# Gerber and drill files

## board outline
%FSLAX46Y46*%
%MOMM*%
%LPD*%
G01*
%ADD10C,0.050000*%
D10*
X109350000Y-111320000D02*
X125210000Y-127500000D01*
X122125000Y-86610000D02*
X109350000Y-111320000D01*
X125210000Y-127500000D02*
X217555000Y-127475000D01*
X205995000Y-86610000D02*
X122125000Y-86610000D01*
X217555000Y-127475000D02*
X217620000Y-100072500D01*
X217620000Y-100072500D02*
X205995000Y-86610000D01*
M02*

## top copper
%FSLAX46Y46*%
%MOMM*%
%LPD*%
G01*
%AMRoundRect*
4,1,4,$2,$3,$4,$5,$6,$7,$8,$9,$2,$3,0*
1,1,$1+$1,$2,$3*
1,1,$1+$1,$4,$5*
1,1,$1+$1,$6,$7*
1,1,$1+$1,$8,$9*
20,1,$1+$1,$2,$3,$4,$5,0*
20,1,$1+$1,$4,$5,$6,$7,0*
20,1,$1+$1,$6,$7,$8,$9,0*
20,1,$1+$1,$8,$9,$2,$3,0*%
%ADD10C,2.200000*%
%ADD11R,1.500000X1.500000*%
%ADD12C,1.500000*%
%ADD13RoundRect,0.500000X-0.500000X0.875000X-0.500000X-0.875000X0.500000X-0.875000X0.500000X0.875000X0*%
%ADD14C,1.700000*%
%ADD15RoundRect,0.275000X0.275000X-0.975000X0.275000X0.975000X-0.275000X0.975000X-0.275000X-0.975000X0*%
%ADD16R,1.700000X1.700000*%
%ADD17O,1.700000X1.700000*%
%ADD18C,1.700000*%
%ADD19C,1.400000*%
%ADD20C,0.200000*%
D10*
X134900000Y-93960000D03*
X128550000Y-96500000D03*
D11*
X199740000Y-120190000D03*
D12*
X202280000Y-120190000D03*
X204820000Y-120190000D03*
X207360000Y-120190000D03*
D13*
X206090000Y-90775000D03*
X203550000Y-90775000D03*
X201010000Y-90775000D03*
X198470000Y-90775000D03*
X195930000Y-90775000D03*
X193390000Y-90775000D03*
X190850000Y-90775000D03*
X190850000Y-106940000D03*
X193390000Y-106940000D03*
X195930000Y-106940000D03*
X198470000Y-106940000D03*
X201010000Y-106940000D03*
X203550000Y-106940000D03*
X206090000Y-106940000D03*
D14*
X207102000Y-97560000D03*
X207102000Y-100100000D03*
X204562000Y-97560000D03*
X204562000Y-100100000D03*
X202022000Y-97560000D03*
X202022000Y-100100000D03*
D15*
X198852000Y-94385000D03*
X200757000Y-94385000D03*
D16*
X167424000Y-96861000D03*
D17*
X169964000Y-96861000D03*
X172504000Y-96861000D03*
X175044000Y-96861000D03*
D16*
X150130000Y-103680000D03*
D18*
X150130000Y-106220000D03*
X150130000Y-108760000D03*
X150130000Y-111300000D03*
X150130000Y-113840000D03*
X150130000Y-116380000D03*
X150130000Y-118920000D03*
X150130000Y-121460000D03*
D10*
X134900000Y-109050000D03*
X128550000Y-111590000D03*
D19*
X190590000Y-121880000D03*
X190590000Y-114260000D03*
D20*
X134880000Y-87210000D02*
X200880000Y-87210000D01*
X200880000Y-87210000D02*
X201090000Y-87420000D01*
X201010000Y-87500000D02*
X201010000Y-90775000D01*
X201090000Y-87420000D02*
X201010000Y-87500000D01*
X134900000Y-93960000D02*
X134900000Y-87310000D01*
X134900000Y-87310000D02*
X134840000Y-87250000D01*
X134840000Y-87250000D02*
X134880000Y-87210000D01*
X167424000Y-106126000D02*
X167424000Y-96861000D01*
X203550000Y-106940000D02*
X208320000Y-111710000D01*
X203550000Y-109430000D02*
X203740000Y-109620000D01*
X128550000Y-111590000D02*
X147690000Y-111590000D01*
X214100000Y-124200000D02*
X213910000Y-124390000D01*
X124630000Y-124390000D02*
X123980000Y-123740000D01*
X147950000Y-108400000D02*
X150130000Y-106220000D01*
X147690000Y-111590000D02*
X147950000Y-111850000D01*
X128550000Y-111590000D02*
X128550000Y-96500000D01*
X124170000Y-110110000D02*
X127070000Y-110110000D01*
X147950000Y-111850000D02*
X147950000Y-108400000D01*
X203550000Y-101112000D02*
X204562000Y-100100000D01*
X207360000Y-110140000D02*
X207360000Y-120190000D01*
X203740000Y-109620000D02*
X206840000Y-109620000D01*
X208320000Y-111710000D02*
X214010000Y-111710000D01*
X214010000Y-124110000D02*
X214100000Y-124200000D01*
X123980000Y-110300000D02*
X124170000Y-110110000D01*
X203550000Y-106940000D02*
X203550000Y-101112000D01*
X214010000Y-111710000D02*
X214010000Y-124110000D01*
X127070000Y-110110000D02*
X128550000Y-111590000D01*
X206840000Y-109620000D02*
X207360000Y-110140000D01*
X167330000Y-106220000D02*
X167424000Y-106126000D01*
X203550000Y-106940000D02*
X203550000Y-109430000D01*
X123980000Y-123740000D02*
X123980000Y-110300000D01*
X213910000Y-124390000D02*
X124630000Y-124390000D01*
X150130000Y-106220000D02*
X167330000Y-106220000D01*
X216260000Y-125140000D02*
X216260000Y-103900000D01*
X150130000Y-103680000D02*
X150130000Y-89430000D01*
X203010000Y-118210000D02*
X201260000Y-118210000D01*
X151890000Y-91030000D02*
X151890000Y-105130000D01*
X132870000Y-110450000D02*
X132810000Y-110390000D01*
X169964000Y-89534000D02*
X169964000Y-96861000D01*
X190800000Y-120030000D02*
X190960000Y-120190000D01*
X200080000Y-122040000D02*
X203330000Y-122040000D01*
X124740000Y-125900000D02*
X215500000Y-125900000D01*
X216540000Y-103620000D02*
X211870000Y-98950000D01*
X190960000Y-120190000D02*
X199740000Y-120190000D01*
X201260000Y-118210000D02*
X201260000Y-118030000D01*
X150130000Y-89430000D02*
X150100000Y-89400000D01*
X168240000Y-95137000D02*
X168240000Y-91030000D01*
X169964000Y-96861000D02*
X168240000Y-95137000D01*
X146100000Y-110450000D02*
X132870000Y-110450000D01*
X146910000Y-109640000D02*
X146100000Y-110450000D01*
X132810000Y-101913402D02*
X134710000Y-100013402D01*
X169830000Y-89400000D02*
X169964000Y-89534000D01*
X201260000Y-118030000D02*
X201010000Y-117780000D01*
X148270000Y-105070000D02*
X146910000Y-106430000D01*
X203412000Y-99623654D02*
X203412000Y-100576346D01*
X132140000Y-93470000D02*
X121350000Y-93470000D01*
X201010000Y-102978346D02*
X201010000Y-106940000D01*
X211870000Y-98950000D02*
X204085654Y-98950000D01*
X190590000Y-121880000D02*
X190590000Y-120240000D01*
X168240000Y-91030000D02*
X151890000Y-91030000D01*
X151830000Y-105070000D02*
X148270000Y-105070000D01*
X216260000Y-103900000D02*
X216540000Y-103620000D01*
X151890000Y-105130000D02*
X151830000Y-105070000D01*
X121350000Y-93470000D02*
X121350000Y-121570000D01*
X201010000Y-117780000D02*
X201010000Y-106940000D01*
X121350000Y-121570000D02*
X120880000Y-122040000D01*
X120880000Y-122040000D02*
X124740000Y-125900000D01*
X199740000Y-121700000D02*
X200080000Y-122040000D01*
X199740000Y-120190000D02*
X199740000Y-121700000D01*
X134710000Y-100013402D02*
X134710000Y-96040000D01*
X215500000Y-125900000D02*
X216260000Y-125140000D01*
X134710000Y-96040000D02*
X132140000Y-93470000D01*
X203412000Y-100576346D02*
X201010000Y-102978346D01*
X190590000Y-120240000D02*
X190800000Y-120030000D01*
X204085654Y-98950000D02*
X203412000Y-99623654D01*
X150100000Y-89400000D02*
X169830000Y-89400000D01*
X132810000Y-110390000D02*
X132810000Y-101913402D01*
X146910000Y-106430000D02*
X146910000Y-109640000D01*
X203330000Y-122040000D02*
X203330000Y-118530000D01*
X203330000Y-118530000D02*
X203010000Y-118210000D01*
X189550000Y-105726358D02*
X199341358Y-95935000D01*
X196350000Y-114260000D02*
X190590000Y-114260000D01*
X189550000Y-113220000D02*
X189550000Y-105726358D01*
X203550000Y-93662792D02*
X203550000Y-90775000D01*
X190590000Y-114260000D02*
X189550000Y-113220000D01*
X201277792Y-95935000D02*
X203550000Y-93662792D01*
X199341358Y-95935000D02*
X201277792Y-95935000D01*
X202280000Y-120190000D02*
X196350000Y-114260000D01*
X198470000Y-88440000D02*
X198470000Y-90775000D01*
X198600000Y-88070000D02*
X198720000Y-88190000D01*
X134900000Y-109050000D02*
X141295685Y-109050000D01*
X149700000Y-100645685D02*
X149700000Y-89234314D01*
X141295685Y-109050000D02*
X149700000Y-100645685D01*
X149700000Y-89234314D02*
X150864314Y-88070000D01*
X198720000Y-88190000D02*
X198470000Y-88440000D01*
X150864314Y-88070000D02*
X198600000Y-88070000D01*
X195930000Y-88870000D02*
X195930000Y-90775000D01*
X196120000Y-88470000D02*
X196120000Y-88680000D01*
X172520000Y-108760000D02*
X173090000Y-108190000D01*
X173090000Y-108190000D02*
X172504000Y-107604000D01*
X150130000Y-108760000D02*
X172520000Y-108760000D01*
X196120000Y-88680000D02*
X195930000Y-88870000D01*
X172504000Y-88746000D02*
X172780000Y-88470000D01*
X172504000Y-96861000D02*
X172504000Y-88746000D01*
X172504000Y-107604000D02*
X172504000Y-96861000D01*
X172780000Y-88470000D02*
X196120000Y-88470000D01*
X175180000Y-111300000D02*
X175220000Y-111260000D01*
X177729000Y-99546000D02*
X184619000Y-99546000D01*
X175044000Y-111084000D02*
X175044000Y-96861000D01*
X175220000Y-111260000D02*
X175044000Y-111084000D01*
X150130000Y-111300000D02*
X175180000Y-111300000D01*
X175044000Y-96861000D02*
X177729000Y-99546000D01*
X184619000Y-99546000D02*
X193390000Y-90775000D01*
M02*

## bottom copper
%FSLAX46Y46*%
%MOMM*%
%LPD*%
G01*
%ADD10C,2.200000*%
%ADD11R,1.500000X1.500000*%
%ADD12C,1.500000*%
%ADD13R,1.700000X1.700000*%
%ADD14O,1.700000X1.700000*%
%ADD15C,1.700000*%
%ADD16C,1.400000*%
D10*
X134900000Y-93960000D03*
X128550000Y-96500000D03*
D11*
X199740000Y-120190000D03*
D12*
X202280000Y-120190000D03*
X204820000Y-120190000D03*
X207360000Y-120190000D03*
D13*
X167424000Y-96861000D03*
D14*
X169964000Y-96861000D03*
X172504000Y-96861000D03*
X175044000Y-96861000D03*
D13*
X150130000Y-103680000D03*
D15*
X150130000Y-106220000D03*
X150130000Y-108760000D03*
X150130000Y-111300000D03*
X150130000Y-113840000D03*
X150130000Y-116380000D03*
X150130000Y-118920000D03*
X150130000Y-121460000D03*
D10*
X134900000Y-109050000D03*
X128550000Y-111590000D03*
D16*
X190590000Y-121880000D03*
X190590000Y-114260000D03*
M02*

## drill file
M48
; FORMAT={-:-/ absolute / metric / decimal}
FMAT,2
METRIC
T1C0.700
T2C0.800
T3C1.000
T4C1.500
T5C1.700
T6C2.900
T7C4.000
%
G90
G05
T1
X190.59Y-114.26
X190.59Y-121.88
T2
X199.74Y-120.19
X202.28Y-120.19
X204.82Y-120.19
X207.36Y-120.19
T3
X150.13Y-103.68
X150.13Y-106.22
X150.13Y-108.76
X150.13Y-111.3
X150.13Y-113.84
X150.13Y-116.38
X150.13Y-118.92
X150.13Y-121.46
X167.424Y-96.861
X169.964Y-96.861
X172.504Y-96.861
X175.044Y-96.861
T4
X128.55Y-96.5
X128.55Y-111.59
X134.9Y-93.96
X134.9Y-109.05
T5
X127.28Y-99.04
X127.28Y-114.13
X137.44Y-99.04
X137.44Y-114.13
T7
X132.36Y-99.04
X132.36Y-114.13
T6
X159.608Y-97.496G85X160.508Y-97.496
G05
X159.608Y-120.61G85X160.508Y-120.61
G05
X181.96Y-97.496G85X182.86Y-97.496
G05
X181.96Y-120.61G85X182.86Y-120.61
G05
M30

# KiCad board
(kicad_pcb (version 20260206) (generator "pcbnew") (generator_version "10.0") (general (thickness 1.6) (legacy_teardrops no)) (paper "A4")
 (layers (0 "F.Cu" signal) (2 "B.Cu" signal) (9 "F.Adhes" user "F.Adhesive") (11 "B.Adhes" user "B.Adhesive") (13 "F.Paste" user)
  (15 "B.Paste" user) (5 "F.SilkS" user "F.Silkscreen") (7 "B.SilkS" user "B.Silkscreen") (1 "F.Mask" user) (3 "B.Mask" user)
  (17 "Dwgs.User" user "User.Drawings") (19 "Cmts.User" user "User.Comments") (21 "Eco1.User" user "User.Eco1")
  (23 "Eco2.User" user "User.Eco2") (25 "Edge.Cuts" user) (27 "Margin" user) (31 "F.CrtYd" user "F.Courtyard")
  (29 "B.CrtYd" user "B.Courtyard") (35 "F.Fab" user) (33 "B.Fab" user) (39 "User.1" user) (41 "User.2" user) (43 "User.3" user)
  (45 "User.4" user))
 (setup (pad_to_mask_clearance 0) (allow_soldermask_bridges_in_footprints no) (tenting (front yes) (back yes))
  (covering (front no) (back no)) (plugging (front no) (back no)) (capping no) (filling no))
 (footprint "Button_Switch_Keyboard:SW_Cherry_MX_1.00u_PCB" (layer "F.Cu") (at 134.9 93.96)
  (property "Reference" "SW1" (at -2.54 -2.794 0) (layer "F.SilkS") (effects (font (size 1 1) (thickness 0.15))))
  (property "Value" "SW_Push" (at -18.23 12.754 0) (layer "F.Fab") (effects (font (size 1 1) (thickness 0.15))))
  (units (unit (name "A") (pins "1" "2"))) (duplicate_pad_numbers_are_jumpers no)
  (pad "" np_thru_hole circle (at -7.62 5.08) (size 1.7 1.7) (drill 1.7) (layers "*.Cu" "*.Mask"))
  (pad "" np_thru_hole circle (at -2.54 5.08) (size 4 4) (drill 4) (layers "*.Cu" "*.Mask"))
  (pad "" np_thru_hole circle (at 2.54 5.08) (size 1.7 1.7) (drill 1.7) (layers "*.Cu" "*.Mask"))
  (pad "1" thru_hole circle (at 0 0) (size 2.2 2.2) (drill 1.5) (layers "*.Cu" "*.Mask") (remove_unused_layers no) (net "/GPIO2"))
  (pad "2" thru_hole circle (at -6.35 2.54) (size 2.2 2.2) (drill 1.5) (layers "*.Cu" "*.Mask") (remove_unused_layers no) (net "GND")))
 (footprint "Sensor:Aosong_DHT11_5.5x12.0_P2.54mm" (layer "F.Cu") (at 199.74 120.19 90)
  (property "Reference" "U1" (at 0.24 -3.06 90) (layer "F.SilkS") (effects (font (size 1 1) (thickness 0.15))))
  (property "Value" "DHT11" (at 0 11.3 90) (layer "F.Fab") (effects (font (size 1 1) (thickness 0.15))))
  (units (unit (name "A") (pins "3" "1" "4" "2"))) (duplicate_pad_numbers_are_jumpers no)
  (pad "1" thru_hole rect (at 0 0 90) (size 1.5 1.5) (drill 0.8) (layers "*.Cu" "*.Mask") (remove_unused_layers no) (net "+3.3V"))
  (pad "2" thru_hole circle (at 0 2.54 90) (size 1.5 1.5) (drill 0.8) (layers "*.Cu" "*.Mask") (remove_unused_layers no) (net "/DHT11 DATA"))
  (pad "3" thru_hole circle (at 0 5.08 90) (size 1.5 1.5) (drill 0.8) (layers "*.Cu" "*.Mask") (remove_unused_layers no)
   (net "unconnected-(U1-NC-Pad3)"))
  (pad "4" thru_hole circle (at 0 7.62 90) (size 1.5 1.5) (drill 0.8) (layers "*.Cu" "*.Mask") (remove_unused_layers no) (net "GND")))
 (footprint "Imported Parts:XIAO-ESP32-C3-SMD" (layer "F.Cu") (at 187.97 89.94 -90)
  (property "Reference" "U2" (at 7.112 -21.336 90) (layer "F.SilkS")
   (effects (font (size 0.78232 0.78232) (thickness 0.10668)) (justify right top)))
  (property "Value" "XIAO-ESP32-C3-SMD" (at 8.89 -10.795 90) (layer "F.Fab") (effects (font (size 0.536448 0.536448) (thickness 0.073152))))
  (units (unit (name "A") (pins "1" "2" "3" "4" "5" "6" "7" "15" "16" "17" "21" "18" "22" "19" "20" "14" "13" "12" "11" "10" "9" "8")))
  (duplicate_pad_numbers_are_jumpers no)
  (pad "1" smd roundrect (at 0.835 -18.12 270) (size 2.75 2) (layers "F.Cu" "F.Mask" "F.Paste") (roundrect_rratio 0.25)
   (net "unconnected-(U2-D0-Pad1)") (solder_mask_margin 0.0508) (thermal_bridge_angle 45))
  (pad "2" smd roundrect (at 0.835 -15.58 270) (size 2.75 2) (layers "F.Cu" "F.Mask" "F.Paste") (roundrect_rratio 0.25) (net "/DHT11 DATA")
   (solder_mask_margin 0.0508) (thermal_bridge_angle 45))
  (pad "3" smd roundrect (at 0.835 -13.04 270) (size 2.75 2) (layers "F.Cu" "F.Mask" "F.Paste") (roundrect_rratio 0.25) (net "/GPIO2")
   (solder_mask_margin 0.0508) (thermal_bridge_angle 45))
  (pad "4" smd roundrect (at 0.835 -10.5 270) (size 2.75 2) (layers "F.Cu" "F.Mask" "F.Paste") (roundrect_rratio 0.25) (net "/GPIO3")
   (solder_mask_margin 0.0508) (thermal_bridge_angle 45))
  (pad "5" smd roundrect (at 0.835 -7.96 270) (size 2.75 2) (layers "F.Cu" "F.Mask" "F.Paste") (roundrect_rratio 0.25) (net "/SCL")
   (solder_mask_margin 0.0508) (thermal_bridge_angle 45))
  (pad "6" smd roundrect (at 0.835 -5.42 270) (size 2.75 2) (layers "F.Cu" "F.Mask" "F.Paste") (roundrect_rratio 0.25) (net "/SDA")
   (solder_mask_margin 0.0508) (thermal_bridge_angle 45))
  (pad "7" smd roundrect (at 0.835 -2.88 270) (size 2.75 2) (layers "F.Cu" "F.Mask" "F.Paste") (roundrect_rratio 0.25)
   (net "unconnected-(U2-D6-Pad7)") (solder_mask_margin 0.0508) (thermal_bridge_angle 45))
  (pad "8" smd roundrect (at 17 -2.88 270) (size 2.75 2) (layers "F.Cu" "F.Mask" "F.Paste") (roundrect_rratio 0.25)
   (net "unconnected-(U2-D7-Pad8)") (solder_mask_margin 0.0508) (thermal_bridge_angle 45))
  (pad "9" smd roundrect (at 17 -5.42 270) (size 2.75 2) (layers "F.Cu" "F.Mask" "F.Paste") (roundrect_rratio 0.25)
   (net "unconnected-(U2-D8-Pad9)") (solder_mask_margin 0.0508) (thermal_bridge_angle 45))
  (pad "10" smd roundrect (at 17 -7.96 270) (size 2.75 2) (layers "F.Cu" "F.Mask" "F.Paste") (roundrect_rratio 0.25)
   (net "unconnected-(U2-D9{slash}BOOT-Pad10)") (solder_mask_margin 0.0508) (thermal_bridge_angle 45))
  (pad "11" smd roundrect (at 17 -10.5 270) (size 2.75 2) (layers "F.Cu" "F.Mask" "F.Paste") (roundrect_rratio 0.25)
   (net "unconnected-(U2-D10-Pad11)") (solder_mask_margin 0.0508) (thermal_bridge_angle 45))
  (pad "12" smd roundrect (at 17 -13.04 270) (size 2.75 2) (layers "F.Cu" "F.Mask" "F.Paste") (roundrect_rratio 0.25) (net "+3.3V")
   (solder_mask_margin 0.0508) (thermal_bridge_angle 45))
  (pad "13" smd roundrect (at 17 -15.58 270) (size 2.75 2) (layers "F.Cu" "F.Mask" "F.Paste") (roundrect_rratio 0.25) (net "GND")
   (solder_mask_margin 0.0508) (thermal_bridge_angle 45))
  (pad "14" smd roundrect (at 17 -18.12 270) (size 2.75 2) (layers "F.Cu" "F.Mask" "F.Paste") (roundrect_rratio 0.25) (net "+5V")
   (solder_mask_margin 0.0508) (thermal_bridge_angle 45))
  (pad "15" smd circle (at 7.62 -19.132 270) (size 1.7 1.7) (layers "F.Cu" "F.Mask" "F.Paste") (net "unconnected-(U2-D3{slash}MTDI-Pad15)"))
  (pad "16" smd circle (at 10.16 -19.132 270) (size 1.7 1.7) (layers "F.Cu" "F.Mask" "F.Paste") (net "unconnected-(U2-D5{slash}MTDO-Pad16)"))
  (pad "17" smd circle (at 7.62 -16.592 270) (size 1.7 1.7) (layers "F.Cu" "F.Mask" "F.Paste") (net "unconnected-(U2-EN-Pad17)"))
  (pad "18" smd circle (at 10.16 -16.592 270) (size 1.7 1.7) (layers "F.Cu" "F.Mask" "F.Paste") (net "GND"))
  (pad "19" smd circle (at 7.62 -14.052 270) (size 1.7 1.7) (layers "F.Cu" "F.Mask" "F.Paste") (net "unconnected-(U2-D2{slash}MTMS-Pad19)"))
  (pad "20" smd circle (at 10.16 -14.052 270) (size 1.7 1.7) (layers "F.Cu" "F.Mask" "F.Paste") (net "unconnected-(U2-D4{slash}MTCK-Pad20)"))
  (pad "21" smd roundrect (at 4.445 -10.882 90) (size 2.5 1.1) (layers "F.Cu" "F.Mask" "F.Paste") (roundrect_rratio 0.25)
   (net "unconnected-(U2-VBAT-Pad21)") (thermal_bridge_angle 45))
  (pad "22" smd roundrect (at 4.445 -12.787 90) (size 2.5 1.1) (layers "F.Cu" "F.Mask" "F.Paste") (roundrect_rratio 0.25)
   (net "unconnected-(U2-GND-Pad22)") (thermal_bridge_angle 45)))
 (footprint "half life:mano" (layer "F.Cu") (at 180.8 111.37)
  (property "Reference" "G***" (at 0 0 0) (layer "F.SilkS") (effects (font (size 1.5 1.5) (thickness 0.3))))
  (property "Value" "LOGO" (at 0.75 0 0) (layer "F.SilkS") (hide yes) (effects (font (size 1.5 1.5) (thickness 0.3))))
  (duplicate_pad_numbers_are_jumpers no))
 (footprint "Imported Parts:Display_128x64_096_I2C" (layer "F.Cu") (at 171.234 96.861)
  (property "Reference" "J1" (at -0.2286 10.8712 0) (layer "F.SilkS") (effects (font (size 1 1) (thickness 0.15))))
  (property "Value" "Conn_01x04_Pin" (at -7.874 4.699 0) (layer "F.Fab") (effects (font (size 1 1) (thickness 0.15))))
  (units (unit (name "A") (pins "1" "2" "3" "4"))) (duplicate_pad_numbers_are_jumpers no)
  (pad "" np_thru_hole oval (at -11.176 0.635) (size 3.8 2.9) (drill oval 3.8 2.9) (layers "*.Cu" "*.Mask"))
  (pad "" np_thru_hole oval (at -11.176 23.749) (size 3.8 2.9) (drill oval 3.8 2.9) (layers "*.Cu" "*.Mask"))
  (pad "" np_thru_hole oval (at 11.176 0.635) (size 3.8 2.9) (drill oval 3.8 2.9) (layers "*.Cu" "*.Mask"))
  (pad "" np_thru_hole oval (at 11.176 23.749) (size 3.8 2.9) (drill oval 3.8 2.9) (layers "*.Cu" "*.Mask"))
  (pad "1" thru_hole rect (at -3.81 0 90) (size 1.7 1.7) (drill 1) (layers "*.Cu" "*.Mask") (remove_unused_layers no) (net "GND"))
  (pad "2" thru_hole oval (at -1.27 0 90) (size 1.7 1.7) (drill 1) (layers "*.Cu" "*.Mask") (remove_unused_layers no) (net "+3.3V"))
  (pad "3" thru_hole oval (at 1.27 0 90) (size 1.7 1.7) (drill 1) (layers "*.Cu" "*.Mask") (remove_unused_layers no) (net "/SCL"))
  (pad "4" thru_hole oval (at 3.81 0 90) (size 1.7 1.7) (drill 1) (layers "*.Cu" "*.Mask") (remove_unused_layers no) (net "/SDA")))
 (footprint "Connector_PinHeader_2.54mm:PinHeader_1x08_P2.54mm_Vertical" (layer "F.Cu") (at 150.13 103.68)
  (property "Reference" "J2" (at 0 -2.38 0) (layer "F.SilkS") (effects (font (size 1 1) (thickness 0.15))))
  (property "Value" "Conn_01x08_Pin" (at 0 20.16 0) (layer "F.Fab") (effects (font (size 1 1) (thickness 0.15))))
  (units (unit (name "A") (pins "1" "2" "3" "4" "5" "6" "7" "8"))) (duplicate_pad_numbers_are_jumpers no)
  (pad "1" thru_hole rect (at 0 0) (size 1.7 1.7) (drill 1) (layers "*.Cu" "*.Mask") (remove_unused_layers no) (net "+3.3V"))
  (pad "2" thru_hole circle (at 0 2.54) (size 1.7 1.7) (drill 1) (layers "*.Cu" "*.Mask") (remove_unused_layers no) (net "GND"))
  (pad "3" thru_hole circle (at 0 5.08) (size 1.7 1.7) (drill 1) (layers "*.Cu" "*.Mask") (remove_unused_layers no) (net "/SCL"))
  (pad "4" thru_hole circle (at 0 7.62) (size 1.7 1.7) (drill 1) (layers "*.Cu" "*.Mask") (remove_unused_layers no) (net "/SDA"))
  (pad "5" thru_hole circle (at 0 10.16) (size 1.7 1.7) (drill 1) (layers "*.Cu" "*.Mask") (remove_unused_layers no)
   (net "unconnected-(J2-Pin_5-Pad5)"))
  (pad "6" thru_hole circle (at 0 12.7) (size 1.7 1.7) (drill 1) (layers "*.Cu" "*.Mask") (remove_unused_layers no)
   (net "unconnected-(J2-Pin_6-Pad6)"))
  (pad "7" thru_hole circle (at 0 15.24) (size 1.7 1.7) (drill 1) (layers "*.Cu" "*.Mask") (remove_unused_layers no)
   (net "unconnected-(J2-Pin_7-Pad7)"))
  (pad "8" thru_hole circle (at 0 17.78) (size 1.7 1.7) (drill 1) (layers "*.Cu" "*.Mask") (remove_unused_layers no)
   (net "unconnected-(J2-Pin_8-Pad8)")))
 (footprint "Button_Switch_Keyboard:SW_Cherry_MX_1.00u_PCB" (layer "F.Cu") (at 134.9 109.05)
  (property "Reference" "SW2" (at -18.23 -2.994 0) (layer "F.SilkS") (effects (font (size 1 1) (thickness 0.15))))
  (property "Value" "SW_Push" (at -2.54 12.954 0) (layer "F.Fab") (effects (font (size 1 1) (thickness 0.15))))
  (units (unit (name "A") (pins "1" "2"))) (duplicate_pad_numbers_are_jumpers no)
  (pad "" np_thru_hole circle (at -7.62 5.08) (size 1.7 1.7) (drill 1.7) (layers "*.Cu" "*.Mask"))
  (pad "" np_thru_hole circle (at -2.54 5.08) (size 4 4) (drill 4) (layers "*.Cu" "*.Mask"))
  (pad "" np_thru_hole circle (at 2.54 5.08) (size 1.7 1.7) (drill 1.7) (layers "*.Cu" "*.Mask"))
  (pad "1" thru_hole circle (at 0 0) (size 2.2 2.2) (drill 1.5) (layers "*.Cu" "*.Mask") (remove_unused_layers no) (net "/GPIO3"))
  (pad "2" thru_hole circle (at -6.35 2.54) (size 2.2 2.2) (drill 1.5) (layers "*.Cu" "*.Mask") (remove_unused_layers no) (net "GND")))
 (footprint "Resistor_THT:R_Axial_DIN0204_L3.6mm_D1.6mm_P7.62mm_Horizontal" (layer "F.Cu") (at 190.59 121.88 90)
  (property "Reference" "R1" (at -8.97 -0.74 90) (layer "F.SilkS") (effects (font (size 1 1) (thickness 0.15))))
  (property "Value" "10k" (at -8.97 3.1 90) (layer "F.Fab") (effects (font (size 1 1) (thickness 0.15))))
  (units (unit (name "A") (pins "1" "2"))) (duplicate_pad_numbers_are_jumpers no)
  (pad "1" thru_hole circle (at 0 0 90) (size 1.4 1.4) (drill 0.7) (layers "*.Cu" "*.Mask") (remove_unused_layers no) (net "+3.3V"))
  (pad "2" thru_hole circle (at 7.62 0 90) (size 1.4 1.4) (drill 0.7) (layers "*.Cu" "*.Mask") (remove_unused_layers no) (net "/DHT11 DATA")))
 (gr_line (start 109.35 111.32) (end 125.21 127.5) (stroke (width 0.05) (type default)) (layer "Edge.Cuts"))
 (gr_line (start 122.125 86.61) (end 109.35 111.32) (stroke (width 0.05) (type default)) (layer "Edge.Cuts"))
 (gr_line (start 125.21 127.5) (end 217.555 127.475) (stroke (width 0.05) (type solid)) (layer "Edge.Cuts"))
 (gr_line (start 205.995 86.61) (end 122.125 86.61) (stroke (width 0.05) (type solid)) (layer "Edge.Cuts"))
 (gr_line (start 217.555 127.475) (end 217.62 100.0725) (stroke (width 0.05) (type solid)) (layer "Edge.Cuts"))
 (gr_line (start 217.62 100.0725) (end 205.995 86.61) (stroke (width 0.05) (type default)) (layer "Edge.Cuts"))
 (segment (start 134.88 87.21) (end 200.88 87.21) (width 0.2) (layer "F.Cu") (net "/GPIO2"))
 (segment (start 200.88 87.21) (end 201.09 87.42) (width 0.2) (layer "F.Cu") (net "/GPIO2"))
 (segment (start 201.01 87.5) (end 201.01 90.775) (width 0.2) (layer "F.Cu") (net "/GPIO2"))
 (segment (start 201.09 87.42) (end 201.01 87.5) (width 0.2) (layer "F.Cu") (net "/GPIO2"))
 (segment (start 134.9 93.96) (end 134.9 87.31) (width 0.2) (layer "F.Cu") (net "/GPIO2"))
 (segment (start 134.9 87.31) (end 134.84 87.25) (width 0.2) (layer "F.Cu") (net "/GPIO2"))
 (segment (start 134.84 87.25) (end 134.88 87.21) (width 0.2) (layer "F.Cu") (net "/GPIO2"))
 (segment (start 167.424 106.126) (end 167.424 96.861) (width 0.2) (layer "F.Cu") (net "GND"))
 (segment (start 203.55 106.94) (end 208.32 111.71) (width 0.2) (layer "F.Cu") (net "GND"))
 (segment (start 203.55 109.43) (end 203.74 109.62) (width 0.2) (layer "F.Cu") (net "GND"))
 (segment (start 128.55 111.59) (end 147.69 111.59) (width 0.2) (layer "F.Cu") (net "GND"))
 (segment (start 214.1 124.2) (end 213.91 124.39) (width 0.2) (layer "F.Cu") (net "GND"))
 (segment (start 124.63 124.39) (end 123.98 123.74) (width 0.2) (layer "F.Cu") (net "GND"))
 (segment (start 147.95 108.4) (end 150.13 106.22) (width 0.2) (layer "F.Cu") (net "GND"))
 (segment (start 147.69 111.59) (end 147.95 111.85) (width 0.2) (layer "F.Cu") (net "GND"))
 (segment (start 128.55 111.59) (end 128.55 96.5) (width 0.2) (layer "F.Cu") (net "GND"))
 (segment (start 124.17 110.11) (end 127.07 110.11) (width 0.2) (layer "F.Cu") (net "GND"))
 (segment (start 147.95 111.85) (end 147.95 108.4) (width 0.2) (layer "F.Cu") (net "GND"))
 (segment (start 203.55 101.112) (end 204.562 100.1) (width 0.2) (layer "F.Cu") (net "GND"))
 (segment (start 207.36 110.14) (end 207.36 120.19) (width 0.2) (layer "F.Cu") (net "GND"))
 (segment (start 203.74 109.62) (end 206.84 109.62) (width 0.2) (layer "F.Cu") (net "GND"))
 (segment (start 208.32 111.71) (end 214.01 111.71) (width 0.2) (layer "F.Cu") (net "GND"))
 (segment (start 214.01 124.11) (end 214.1 124.2) (width 0.2) (layer "F.Cu") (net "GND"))
 (segment (start 123.98 110.3) (end 124.17 110.11) (width 0.2) (layer "F.Cu") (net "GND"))
 (segment (start 203.55 106.94) (end 203.55 101.112) (width 0.2) (layer "F.Cu") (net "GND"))
 (segment (start 214.01 111.71) (end 214.01 124.11) (width 0.2) (layer "F.Cu") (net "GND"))
 (segment (start 127.07 110.11) (end 128.55 111.59) (width 0.2) (layer "F.Cu") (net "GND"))
 (segment (start 206.84 109.62) (end 207.36 110.14) (width 0.2) (layer "F.Cu") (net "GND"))
 (segment (start 167.33 106.22) (end 167.424 106.126) (width 0.2) (layer "F.Cu") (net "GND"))
 (segment (start 203.55 106.94) (end 203.55 109.43) (width 0.2) (layer "F.Cu") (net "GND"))
 (segment (start 123.98 123.74) (end 123.98 110.3) (width 0.2) (layer "F.Cu") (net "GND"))
 (segment (start 213.91 124.39) (end 124.63 124.39) (width 0.2) (layer "F.Cu") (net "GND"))
 (segment (start 150.13 106.22) (end 167.33 106.22) (width 0.2) (layer "F.Cu") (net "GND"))
 (segment (start 216.26 125.14) (end 216.26 103.9) (width 0.2) (layer "F.Cu") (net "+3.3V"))
 (segment (start 150.13 103.68) (end 150.13 89.43) (width 0.2) (layer "F.Cu") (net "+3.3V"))
 (segment (start 203.01 118.21) (end 201.26 118.21) (width 0.2) (layer "F.Cu") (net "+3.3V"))
 (segment (start 151.89 91.03) (end 151.89 105.13) (width 0.2) (layer "F.Cu") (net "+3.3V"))
 (segment (start 132.87 110.45) (end 132.81 110.39) (width 0.2) (layer "F.Cu") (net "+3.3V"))
 (segment (start 169.964 89.534) (end 169.964 96.861) (width 0.2) (layer "F.Cu") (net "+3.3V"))
 (segment (start 190.8 120.03) (end 190.96 120.19) (width 0.2) (layer "F.Cu") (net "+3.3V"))
 (segment (start 200.08 122.04) (end 203.33 122.04) (width 0.2) (layer "F.Cu") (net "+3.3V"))
 (segment (start 124.74 125.9) (end 215.5 125.9) (width 0.2) (layer "F.Cu") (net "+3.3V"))
 (segment (start 216.54 103.62) (end 211.87 98.95) (width 0.2) (layer "F.Cu") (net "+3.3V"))
 (segment (start 190.96 120.19) (end 199.74 120.19) (width 0.2) (layer "F.Cu") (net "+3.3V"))
 (segment (start 201.26 118.21) (end 201.26 118.03) (width 0.2) (layer "F.Cu") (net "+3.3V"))
 (segment (start 150.13 89.43) (end 150.1 89.4) (width 0.2) (layer "F.Cu") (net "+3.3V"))
 (segment (start 168.24 95.137) (end 168.24 91.03) (width 0.2) (layer "F.Cu") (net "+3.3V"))
 (segment (start 169.964 96.861) (end 168.24 95.137) (width 0.2) (layer "F.Cu") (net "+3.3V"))
 (segment (start 146.1 110.45) (end 132.87 110.45) (width 0.2) (layer "F.Cu") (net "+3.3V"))
 (segment (start 146.91 109.64) (end 146.1 110.45) (width 0.2) (layer "F.Cu") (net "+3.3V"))
 (segment (start 132.81 101.913402) (end 134.71 100.013402) (width 0.2) (layer "F.Cu") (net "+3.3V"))
 (segment (start 169.83 89.4) (end 169.964 89.534) (width 0.2) (layer "F.Cu") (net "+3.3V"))
 (segment (start 201.26 118.03) (end 201.01 117.78) (width 0.2) (layer "F.Cu") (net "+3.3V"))
 (segment (start 148.27 105.07) (end 146.91 106.43) (width 0.2) (layer "F.Cu") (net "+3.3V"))
 (segment (start 203.412 99.623654) (end 203.412 100.576346) (width 0.2) (layer "F.Cu") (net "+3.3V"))
 (segment (start 132.14 93.47) (end 121.35 93.47) (width 0.2) (layer "F.Cu") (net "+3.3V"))
 (segment (start 201.01 102.978346) (end 201.01 106.94) (width 0.2) (layer "F.Cu") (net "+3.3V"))
 (segment (start 211.87 98.95) (end 204.085654 98.95) (width 0.2) (layer "F.Cu") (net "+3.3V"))
 (segment (start 190.59 121.88) (end 190.59 120.24) (width 0.2) (layer "F.Cu") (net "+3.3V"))
 (segment (start 168.24 91.03) (end 151.89 91.03) (width 0.2) (layer "F.Cu") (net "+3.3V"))
 (segment (start 151.83 105.07) (end 148.27 105.07) (width 0.2) (layer "F.Cu") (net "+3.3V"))
 (segment (start 216.26 103.9) (end 216.54 103.62) (width 0.2) (layer "F.Cu") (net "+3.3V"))
 (segment (start 151.89 105.13) (end 151.83 105.07) (width 0.2) (layer "F.Cu") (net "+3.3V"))
 (segment (start 121.35 93.47) (end 121.35 121.57) (width 0.2) (layer "F.Cu") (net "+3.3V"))
 (segment (start 201.01 117.78) (end 201.01 106.94) (width 0.2) (layer "F.Cu") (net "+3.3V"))
 (segment (start 121.35 121.57) (end 120.88 122.04) (width 0.2) (layer "F.Cu") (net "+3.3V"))
 (segment (start 120.88 122.04) (end 124.74 125.9) (width 0.2) (layer "F.Cu") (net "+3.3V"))
 (segment (start 199.74 121.7) (end 200.08 122.04) (width 0.2) (layer "F.Cu") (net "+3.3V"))
 (segment (start 199.74 120.19) (end 199.74 121.7) (width 0.2) (layer "F.Cu") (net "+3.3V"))
 (segment (start 134.71 100.013402) (end 134.71 96.04) (width 0.2) (layer "F.Cu") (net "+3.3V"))
 (segment (start 215.5 125.9) (end 216.26 125.14) (width 0.2) (layer "F.Cu") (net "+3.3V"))
 (segment (start 134.71 96.04) (end 132.14 93.47) (width 0.2) (layer "F.Cu") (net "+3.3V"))
 (segment (start 203.412 100.576346) (end 201.01 102.978346) (width 0.2) (layer "F.Cu") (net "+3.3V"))
 (segment (start 190.59 120.24) (end 190.8 120.03) (width 0.2) (layer "F.Cu") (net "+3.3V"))
 (segment (start 204.085654 98.95) (end 203.412 99.623654) (width 0.2) (layer "F.Cu") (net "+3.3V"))
 (segment (start 150.1 89.4) (end 169.83 89.4) (width 0.2) (layer "F.Cu") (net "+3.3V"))
 (segment (start 132.81 110.39) (end 132.81 101.913402) (width 0.2) (layer "F.Cu") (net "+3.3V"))
 (segment (start 146.91 106.43) (end 146.91 109.64) (width 0.2) (layer "F.Cu") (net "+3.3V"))
 (segment (start 203.33 122.04) (end 203.33 118.53) (width 0.2) (layer "F.Cu") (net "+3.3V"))
 (segment (start 203.33 118.53) (end 203.01 118.21) (width 0.2) (layer "F.Cu") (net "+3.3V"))
 (segment (start 189.55 105.726358) (end 199.341358 95.935) (width 0.2) (layer "F.Cu") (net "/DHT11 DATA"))
 (segment (start 196.35 114.26) (end 190.59 114.26) (width 0.2) (layer "F.Cu") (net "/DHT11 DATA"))
 (segment (start 189.55 113.22) (end 189.55 105.726358) (width 0.2) (layer "F.Cu") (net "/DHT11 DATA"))
 (segment (start 203.55 93.662792) (end 203.55 90.775) (width 0.2) (layer "F.Cu") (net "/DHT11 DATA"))
 (segment (start 190.59 114.26) (end 189.55 113.22) (width 0.2) (layer "F.Cu") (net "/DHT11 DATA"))
 (segment (start 201.277792 95.935) (end 203.55 93.662792) (width 0.2) (layer "F.Cu") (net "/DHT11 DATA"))
 (segment (start 199.341358 95.935) (end 201.277792 95.935) (width 0.2) (layer "F.Cu") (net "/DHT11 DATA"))
 (segment (start 202.28 120.19) (end 196.35 114.26) (width 0.2) (layer "F.Cu") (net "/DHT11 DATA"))
 (segment (start 198.47 88.44) (end 198.47 90.775) (width 0.2) (layer "F.Cu") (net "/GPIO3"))
 (segment (start 198.6 88.07) (end 198.72 88.19) (width 0.2) (layer "F.Cu") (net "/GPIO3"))
 (segment (start 134.9 109.05) (end 141.295685 109.05) (width 0.2) (layer "F.Cu") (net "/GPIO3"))
 (segment (start 149.7 100.645685) (end 149.7 89.234314) (width 0.2) (layer "F.Cu") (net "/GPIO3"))
 (segment (start 141.295685 109.05) (end 149.7 100.645685) (width 0.2) (layer "F.Cu") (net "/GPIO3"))
 (segment (start 149.7 89.234314) (end 150.864314 88.07) (width 0.2) (layer "F.Cu") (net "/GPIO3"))
 (segment (start 198.72 88.19) (end 198.47 88.44) (width 0.2) (layer "F.Cu") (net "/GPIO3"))
 (segment (start 150.864314 88.07) (end 198.6 88.07) (width 0.2) (layer "F.Cu") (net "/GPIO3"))
 (segment (start 195.93 88.87) (end 195.93 90.775) (width 0.2) (layer "F.Cu") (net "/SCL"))
 (segment (start 196.12 88.47) (end 196.12 88.68) (width 0.2) (layer "F.Cu") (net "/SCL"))
 (segment (start 172.52 108.76) (end 173.09 108.19) (width 0.2) (layer "F.Cu") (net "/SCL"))
 (segment (start 173.09 108.19) (end 172.504 107.604) (width 0.2) (layer "F.Cu") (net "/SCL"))
 (segment (start 150.13 108.76) (end 172.52 108.76) (width 0.2) (layer "F.Cu") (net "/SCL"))
 (segment (start 196.12 88.68) (end 195.93 88.87) (width 0.2) (layer "F.Cu") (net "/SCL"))
 (segment (start 172.504 88.746) (end 172.78 88.47) (width 0.2) (layer "F.Cu") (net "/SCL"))
 (segment (start 172.504 96.861) (end 172.504 88.746) (width 0.2) (layer "F.Cu") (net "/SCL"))
 (segment (start 172.504 107.604) (end 172.504 96.861) (width 0.2) (layer "F.Cu") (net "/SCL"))
 (segment (start 172.78 88.47) (end 196.12 88.47) (width 0.2) (layer "F.Cu") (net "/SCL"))
 (segment (start 175.18 111.3) (end 175.22 111.26) (width 0.2) (layer "F.Cu") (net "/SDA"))
 (segment (start 177.729 99.546) (end 184.619 99.546) (width 0.2) (layer "F.Cu") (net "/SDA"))
 (segment (start 175.044 111.084) (end 175.044 96.861) (width 0.2) (layer "F.Cu") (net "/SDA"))
 (segment (start 175.22 111.26) (end 175.044 111.084) (width 0.2) (layer "F.Cu") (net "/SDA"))
 (segment (start 150.13 111.3) (end 175.18 111.3) (width 0.2) (layer "F.Cu") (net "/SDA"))
 (segment (start 175.044 96.861) (end 177.729 99.546) (width 0.2) (layer "F.Cu") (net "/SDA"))
 (segment (start 184.619 99.546) (end 193.39 90.775) (width 0.2) (layer "F.Cu") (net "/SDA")))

